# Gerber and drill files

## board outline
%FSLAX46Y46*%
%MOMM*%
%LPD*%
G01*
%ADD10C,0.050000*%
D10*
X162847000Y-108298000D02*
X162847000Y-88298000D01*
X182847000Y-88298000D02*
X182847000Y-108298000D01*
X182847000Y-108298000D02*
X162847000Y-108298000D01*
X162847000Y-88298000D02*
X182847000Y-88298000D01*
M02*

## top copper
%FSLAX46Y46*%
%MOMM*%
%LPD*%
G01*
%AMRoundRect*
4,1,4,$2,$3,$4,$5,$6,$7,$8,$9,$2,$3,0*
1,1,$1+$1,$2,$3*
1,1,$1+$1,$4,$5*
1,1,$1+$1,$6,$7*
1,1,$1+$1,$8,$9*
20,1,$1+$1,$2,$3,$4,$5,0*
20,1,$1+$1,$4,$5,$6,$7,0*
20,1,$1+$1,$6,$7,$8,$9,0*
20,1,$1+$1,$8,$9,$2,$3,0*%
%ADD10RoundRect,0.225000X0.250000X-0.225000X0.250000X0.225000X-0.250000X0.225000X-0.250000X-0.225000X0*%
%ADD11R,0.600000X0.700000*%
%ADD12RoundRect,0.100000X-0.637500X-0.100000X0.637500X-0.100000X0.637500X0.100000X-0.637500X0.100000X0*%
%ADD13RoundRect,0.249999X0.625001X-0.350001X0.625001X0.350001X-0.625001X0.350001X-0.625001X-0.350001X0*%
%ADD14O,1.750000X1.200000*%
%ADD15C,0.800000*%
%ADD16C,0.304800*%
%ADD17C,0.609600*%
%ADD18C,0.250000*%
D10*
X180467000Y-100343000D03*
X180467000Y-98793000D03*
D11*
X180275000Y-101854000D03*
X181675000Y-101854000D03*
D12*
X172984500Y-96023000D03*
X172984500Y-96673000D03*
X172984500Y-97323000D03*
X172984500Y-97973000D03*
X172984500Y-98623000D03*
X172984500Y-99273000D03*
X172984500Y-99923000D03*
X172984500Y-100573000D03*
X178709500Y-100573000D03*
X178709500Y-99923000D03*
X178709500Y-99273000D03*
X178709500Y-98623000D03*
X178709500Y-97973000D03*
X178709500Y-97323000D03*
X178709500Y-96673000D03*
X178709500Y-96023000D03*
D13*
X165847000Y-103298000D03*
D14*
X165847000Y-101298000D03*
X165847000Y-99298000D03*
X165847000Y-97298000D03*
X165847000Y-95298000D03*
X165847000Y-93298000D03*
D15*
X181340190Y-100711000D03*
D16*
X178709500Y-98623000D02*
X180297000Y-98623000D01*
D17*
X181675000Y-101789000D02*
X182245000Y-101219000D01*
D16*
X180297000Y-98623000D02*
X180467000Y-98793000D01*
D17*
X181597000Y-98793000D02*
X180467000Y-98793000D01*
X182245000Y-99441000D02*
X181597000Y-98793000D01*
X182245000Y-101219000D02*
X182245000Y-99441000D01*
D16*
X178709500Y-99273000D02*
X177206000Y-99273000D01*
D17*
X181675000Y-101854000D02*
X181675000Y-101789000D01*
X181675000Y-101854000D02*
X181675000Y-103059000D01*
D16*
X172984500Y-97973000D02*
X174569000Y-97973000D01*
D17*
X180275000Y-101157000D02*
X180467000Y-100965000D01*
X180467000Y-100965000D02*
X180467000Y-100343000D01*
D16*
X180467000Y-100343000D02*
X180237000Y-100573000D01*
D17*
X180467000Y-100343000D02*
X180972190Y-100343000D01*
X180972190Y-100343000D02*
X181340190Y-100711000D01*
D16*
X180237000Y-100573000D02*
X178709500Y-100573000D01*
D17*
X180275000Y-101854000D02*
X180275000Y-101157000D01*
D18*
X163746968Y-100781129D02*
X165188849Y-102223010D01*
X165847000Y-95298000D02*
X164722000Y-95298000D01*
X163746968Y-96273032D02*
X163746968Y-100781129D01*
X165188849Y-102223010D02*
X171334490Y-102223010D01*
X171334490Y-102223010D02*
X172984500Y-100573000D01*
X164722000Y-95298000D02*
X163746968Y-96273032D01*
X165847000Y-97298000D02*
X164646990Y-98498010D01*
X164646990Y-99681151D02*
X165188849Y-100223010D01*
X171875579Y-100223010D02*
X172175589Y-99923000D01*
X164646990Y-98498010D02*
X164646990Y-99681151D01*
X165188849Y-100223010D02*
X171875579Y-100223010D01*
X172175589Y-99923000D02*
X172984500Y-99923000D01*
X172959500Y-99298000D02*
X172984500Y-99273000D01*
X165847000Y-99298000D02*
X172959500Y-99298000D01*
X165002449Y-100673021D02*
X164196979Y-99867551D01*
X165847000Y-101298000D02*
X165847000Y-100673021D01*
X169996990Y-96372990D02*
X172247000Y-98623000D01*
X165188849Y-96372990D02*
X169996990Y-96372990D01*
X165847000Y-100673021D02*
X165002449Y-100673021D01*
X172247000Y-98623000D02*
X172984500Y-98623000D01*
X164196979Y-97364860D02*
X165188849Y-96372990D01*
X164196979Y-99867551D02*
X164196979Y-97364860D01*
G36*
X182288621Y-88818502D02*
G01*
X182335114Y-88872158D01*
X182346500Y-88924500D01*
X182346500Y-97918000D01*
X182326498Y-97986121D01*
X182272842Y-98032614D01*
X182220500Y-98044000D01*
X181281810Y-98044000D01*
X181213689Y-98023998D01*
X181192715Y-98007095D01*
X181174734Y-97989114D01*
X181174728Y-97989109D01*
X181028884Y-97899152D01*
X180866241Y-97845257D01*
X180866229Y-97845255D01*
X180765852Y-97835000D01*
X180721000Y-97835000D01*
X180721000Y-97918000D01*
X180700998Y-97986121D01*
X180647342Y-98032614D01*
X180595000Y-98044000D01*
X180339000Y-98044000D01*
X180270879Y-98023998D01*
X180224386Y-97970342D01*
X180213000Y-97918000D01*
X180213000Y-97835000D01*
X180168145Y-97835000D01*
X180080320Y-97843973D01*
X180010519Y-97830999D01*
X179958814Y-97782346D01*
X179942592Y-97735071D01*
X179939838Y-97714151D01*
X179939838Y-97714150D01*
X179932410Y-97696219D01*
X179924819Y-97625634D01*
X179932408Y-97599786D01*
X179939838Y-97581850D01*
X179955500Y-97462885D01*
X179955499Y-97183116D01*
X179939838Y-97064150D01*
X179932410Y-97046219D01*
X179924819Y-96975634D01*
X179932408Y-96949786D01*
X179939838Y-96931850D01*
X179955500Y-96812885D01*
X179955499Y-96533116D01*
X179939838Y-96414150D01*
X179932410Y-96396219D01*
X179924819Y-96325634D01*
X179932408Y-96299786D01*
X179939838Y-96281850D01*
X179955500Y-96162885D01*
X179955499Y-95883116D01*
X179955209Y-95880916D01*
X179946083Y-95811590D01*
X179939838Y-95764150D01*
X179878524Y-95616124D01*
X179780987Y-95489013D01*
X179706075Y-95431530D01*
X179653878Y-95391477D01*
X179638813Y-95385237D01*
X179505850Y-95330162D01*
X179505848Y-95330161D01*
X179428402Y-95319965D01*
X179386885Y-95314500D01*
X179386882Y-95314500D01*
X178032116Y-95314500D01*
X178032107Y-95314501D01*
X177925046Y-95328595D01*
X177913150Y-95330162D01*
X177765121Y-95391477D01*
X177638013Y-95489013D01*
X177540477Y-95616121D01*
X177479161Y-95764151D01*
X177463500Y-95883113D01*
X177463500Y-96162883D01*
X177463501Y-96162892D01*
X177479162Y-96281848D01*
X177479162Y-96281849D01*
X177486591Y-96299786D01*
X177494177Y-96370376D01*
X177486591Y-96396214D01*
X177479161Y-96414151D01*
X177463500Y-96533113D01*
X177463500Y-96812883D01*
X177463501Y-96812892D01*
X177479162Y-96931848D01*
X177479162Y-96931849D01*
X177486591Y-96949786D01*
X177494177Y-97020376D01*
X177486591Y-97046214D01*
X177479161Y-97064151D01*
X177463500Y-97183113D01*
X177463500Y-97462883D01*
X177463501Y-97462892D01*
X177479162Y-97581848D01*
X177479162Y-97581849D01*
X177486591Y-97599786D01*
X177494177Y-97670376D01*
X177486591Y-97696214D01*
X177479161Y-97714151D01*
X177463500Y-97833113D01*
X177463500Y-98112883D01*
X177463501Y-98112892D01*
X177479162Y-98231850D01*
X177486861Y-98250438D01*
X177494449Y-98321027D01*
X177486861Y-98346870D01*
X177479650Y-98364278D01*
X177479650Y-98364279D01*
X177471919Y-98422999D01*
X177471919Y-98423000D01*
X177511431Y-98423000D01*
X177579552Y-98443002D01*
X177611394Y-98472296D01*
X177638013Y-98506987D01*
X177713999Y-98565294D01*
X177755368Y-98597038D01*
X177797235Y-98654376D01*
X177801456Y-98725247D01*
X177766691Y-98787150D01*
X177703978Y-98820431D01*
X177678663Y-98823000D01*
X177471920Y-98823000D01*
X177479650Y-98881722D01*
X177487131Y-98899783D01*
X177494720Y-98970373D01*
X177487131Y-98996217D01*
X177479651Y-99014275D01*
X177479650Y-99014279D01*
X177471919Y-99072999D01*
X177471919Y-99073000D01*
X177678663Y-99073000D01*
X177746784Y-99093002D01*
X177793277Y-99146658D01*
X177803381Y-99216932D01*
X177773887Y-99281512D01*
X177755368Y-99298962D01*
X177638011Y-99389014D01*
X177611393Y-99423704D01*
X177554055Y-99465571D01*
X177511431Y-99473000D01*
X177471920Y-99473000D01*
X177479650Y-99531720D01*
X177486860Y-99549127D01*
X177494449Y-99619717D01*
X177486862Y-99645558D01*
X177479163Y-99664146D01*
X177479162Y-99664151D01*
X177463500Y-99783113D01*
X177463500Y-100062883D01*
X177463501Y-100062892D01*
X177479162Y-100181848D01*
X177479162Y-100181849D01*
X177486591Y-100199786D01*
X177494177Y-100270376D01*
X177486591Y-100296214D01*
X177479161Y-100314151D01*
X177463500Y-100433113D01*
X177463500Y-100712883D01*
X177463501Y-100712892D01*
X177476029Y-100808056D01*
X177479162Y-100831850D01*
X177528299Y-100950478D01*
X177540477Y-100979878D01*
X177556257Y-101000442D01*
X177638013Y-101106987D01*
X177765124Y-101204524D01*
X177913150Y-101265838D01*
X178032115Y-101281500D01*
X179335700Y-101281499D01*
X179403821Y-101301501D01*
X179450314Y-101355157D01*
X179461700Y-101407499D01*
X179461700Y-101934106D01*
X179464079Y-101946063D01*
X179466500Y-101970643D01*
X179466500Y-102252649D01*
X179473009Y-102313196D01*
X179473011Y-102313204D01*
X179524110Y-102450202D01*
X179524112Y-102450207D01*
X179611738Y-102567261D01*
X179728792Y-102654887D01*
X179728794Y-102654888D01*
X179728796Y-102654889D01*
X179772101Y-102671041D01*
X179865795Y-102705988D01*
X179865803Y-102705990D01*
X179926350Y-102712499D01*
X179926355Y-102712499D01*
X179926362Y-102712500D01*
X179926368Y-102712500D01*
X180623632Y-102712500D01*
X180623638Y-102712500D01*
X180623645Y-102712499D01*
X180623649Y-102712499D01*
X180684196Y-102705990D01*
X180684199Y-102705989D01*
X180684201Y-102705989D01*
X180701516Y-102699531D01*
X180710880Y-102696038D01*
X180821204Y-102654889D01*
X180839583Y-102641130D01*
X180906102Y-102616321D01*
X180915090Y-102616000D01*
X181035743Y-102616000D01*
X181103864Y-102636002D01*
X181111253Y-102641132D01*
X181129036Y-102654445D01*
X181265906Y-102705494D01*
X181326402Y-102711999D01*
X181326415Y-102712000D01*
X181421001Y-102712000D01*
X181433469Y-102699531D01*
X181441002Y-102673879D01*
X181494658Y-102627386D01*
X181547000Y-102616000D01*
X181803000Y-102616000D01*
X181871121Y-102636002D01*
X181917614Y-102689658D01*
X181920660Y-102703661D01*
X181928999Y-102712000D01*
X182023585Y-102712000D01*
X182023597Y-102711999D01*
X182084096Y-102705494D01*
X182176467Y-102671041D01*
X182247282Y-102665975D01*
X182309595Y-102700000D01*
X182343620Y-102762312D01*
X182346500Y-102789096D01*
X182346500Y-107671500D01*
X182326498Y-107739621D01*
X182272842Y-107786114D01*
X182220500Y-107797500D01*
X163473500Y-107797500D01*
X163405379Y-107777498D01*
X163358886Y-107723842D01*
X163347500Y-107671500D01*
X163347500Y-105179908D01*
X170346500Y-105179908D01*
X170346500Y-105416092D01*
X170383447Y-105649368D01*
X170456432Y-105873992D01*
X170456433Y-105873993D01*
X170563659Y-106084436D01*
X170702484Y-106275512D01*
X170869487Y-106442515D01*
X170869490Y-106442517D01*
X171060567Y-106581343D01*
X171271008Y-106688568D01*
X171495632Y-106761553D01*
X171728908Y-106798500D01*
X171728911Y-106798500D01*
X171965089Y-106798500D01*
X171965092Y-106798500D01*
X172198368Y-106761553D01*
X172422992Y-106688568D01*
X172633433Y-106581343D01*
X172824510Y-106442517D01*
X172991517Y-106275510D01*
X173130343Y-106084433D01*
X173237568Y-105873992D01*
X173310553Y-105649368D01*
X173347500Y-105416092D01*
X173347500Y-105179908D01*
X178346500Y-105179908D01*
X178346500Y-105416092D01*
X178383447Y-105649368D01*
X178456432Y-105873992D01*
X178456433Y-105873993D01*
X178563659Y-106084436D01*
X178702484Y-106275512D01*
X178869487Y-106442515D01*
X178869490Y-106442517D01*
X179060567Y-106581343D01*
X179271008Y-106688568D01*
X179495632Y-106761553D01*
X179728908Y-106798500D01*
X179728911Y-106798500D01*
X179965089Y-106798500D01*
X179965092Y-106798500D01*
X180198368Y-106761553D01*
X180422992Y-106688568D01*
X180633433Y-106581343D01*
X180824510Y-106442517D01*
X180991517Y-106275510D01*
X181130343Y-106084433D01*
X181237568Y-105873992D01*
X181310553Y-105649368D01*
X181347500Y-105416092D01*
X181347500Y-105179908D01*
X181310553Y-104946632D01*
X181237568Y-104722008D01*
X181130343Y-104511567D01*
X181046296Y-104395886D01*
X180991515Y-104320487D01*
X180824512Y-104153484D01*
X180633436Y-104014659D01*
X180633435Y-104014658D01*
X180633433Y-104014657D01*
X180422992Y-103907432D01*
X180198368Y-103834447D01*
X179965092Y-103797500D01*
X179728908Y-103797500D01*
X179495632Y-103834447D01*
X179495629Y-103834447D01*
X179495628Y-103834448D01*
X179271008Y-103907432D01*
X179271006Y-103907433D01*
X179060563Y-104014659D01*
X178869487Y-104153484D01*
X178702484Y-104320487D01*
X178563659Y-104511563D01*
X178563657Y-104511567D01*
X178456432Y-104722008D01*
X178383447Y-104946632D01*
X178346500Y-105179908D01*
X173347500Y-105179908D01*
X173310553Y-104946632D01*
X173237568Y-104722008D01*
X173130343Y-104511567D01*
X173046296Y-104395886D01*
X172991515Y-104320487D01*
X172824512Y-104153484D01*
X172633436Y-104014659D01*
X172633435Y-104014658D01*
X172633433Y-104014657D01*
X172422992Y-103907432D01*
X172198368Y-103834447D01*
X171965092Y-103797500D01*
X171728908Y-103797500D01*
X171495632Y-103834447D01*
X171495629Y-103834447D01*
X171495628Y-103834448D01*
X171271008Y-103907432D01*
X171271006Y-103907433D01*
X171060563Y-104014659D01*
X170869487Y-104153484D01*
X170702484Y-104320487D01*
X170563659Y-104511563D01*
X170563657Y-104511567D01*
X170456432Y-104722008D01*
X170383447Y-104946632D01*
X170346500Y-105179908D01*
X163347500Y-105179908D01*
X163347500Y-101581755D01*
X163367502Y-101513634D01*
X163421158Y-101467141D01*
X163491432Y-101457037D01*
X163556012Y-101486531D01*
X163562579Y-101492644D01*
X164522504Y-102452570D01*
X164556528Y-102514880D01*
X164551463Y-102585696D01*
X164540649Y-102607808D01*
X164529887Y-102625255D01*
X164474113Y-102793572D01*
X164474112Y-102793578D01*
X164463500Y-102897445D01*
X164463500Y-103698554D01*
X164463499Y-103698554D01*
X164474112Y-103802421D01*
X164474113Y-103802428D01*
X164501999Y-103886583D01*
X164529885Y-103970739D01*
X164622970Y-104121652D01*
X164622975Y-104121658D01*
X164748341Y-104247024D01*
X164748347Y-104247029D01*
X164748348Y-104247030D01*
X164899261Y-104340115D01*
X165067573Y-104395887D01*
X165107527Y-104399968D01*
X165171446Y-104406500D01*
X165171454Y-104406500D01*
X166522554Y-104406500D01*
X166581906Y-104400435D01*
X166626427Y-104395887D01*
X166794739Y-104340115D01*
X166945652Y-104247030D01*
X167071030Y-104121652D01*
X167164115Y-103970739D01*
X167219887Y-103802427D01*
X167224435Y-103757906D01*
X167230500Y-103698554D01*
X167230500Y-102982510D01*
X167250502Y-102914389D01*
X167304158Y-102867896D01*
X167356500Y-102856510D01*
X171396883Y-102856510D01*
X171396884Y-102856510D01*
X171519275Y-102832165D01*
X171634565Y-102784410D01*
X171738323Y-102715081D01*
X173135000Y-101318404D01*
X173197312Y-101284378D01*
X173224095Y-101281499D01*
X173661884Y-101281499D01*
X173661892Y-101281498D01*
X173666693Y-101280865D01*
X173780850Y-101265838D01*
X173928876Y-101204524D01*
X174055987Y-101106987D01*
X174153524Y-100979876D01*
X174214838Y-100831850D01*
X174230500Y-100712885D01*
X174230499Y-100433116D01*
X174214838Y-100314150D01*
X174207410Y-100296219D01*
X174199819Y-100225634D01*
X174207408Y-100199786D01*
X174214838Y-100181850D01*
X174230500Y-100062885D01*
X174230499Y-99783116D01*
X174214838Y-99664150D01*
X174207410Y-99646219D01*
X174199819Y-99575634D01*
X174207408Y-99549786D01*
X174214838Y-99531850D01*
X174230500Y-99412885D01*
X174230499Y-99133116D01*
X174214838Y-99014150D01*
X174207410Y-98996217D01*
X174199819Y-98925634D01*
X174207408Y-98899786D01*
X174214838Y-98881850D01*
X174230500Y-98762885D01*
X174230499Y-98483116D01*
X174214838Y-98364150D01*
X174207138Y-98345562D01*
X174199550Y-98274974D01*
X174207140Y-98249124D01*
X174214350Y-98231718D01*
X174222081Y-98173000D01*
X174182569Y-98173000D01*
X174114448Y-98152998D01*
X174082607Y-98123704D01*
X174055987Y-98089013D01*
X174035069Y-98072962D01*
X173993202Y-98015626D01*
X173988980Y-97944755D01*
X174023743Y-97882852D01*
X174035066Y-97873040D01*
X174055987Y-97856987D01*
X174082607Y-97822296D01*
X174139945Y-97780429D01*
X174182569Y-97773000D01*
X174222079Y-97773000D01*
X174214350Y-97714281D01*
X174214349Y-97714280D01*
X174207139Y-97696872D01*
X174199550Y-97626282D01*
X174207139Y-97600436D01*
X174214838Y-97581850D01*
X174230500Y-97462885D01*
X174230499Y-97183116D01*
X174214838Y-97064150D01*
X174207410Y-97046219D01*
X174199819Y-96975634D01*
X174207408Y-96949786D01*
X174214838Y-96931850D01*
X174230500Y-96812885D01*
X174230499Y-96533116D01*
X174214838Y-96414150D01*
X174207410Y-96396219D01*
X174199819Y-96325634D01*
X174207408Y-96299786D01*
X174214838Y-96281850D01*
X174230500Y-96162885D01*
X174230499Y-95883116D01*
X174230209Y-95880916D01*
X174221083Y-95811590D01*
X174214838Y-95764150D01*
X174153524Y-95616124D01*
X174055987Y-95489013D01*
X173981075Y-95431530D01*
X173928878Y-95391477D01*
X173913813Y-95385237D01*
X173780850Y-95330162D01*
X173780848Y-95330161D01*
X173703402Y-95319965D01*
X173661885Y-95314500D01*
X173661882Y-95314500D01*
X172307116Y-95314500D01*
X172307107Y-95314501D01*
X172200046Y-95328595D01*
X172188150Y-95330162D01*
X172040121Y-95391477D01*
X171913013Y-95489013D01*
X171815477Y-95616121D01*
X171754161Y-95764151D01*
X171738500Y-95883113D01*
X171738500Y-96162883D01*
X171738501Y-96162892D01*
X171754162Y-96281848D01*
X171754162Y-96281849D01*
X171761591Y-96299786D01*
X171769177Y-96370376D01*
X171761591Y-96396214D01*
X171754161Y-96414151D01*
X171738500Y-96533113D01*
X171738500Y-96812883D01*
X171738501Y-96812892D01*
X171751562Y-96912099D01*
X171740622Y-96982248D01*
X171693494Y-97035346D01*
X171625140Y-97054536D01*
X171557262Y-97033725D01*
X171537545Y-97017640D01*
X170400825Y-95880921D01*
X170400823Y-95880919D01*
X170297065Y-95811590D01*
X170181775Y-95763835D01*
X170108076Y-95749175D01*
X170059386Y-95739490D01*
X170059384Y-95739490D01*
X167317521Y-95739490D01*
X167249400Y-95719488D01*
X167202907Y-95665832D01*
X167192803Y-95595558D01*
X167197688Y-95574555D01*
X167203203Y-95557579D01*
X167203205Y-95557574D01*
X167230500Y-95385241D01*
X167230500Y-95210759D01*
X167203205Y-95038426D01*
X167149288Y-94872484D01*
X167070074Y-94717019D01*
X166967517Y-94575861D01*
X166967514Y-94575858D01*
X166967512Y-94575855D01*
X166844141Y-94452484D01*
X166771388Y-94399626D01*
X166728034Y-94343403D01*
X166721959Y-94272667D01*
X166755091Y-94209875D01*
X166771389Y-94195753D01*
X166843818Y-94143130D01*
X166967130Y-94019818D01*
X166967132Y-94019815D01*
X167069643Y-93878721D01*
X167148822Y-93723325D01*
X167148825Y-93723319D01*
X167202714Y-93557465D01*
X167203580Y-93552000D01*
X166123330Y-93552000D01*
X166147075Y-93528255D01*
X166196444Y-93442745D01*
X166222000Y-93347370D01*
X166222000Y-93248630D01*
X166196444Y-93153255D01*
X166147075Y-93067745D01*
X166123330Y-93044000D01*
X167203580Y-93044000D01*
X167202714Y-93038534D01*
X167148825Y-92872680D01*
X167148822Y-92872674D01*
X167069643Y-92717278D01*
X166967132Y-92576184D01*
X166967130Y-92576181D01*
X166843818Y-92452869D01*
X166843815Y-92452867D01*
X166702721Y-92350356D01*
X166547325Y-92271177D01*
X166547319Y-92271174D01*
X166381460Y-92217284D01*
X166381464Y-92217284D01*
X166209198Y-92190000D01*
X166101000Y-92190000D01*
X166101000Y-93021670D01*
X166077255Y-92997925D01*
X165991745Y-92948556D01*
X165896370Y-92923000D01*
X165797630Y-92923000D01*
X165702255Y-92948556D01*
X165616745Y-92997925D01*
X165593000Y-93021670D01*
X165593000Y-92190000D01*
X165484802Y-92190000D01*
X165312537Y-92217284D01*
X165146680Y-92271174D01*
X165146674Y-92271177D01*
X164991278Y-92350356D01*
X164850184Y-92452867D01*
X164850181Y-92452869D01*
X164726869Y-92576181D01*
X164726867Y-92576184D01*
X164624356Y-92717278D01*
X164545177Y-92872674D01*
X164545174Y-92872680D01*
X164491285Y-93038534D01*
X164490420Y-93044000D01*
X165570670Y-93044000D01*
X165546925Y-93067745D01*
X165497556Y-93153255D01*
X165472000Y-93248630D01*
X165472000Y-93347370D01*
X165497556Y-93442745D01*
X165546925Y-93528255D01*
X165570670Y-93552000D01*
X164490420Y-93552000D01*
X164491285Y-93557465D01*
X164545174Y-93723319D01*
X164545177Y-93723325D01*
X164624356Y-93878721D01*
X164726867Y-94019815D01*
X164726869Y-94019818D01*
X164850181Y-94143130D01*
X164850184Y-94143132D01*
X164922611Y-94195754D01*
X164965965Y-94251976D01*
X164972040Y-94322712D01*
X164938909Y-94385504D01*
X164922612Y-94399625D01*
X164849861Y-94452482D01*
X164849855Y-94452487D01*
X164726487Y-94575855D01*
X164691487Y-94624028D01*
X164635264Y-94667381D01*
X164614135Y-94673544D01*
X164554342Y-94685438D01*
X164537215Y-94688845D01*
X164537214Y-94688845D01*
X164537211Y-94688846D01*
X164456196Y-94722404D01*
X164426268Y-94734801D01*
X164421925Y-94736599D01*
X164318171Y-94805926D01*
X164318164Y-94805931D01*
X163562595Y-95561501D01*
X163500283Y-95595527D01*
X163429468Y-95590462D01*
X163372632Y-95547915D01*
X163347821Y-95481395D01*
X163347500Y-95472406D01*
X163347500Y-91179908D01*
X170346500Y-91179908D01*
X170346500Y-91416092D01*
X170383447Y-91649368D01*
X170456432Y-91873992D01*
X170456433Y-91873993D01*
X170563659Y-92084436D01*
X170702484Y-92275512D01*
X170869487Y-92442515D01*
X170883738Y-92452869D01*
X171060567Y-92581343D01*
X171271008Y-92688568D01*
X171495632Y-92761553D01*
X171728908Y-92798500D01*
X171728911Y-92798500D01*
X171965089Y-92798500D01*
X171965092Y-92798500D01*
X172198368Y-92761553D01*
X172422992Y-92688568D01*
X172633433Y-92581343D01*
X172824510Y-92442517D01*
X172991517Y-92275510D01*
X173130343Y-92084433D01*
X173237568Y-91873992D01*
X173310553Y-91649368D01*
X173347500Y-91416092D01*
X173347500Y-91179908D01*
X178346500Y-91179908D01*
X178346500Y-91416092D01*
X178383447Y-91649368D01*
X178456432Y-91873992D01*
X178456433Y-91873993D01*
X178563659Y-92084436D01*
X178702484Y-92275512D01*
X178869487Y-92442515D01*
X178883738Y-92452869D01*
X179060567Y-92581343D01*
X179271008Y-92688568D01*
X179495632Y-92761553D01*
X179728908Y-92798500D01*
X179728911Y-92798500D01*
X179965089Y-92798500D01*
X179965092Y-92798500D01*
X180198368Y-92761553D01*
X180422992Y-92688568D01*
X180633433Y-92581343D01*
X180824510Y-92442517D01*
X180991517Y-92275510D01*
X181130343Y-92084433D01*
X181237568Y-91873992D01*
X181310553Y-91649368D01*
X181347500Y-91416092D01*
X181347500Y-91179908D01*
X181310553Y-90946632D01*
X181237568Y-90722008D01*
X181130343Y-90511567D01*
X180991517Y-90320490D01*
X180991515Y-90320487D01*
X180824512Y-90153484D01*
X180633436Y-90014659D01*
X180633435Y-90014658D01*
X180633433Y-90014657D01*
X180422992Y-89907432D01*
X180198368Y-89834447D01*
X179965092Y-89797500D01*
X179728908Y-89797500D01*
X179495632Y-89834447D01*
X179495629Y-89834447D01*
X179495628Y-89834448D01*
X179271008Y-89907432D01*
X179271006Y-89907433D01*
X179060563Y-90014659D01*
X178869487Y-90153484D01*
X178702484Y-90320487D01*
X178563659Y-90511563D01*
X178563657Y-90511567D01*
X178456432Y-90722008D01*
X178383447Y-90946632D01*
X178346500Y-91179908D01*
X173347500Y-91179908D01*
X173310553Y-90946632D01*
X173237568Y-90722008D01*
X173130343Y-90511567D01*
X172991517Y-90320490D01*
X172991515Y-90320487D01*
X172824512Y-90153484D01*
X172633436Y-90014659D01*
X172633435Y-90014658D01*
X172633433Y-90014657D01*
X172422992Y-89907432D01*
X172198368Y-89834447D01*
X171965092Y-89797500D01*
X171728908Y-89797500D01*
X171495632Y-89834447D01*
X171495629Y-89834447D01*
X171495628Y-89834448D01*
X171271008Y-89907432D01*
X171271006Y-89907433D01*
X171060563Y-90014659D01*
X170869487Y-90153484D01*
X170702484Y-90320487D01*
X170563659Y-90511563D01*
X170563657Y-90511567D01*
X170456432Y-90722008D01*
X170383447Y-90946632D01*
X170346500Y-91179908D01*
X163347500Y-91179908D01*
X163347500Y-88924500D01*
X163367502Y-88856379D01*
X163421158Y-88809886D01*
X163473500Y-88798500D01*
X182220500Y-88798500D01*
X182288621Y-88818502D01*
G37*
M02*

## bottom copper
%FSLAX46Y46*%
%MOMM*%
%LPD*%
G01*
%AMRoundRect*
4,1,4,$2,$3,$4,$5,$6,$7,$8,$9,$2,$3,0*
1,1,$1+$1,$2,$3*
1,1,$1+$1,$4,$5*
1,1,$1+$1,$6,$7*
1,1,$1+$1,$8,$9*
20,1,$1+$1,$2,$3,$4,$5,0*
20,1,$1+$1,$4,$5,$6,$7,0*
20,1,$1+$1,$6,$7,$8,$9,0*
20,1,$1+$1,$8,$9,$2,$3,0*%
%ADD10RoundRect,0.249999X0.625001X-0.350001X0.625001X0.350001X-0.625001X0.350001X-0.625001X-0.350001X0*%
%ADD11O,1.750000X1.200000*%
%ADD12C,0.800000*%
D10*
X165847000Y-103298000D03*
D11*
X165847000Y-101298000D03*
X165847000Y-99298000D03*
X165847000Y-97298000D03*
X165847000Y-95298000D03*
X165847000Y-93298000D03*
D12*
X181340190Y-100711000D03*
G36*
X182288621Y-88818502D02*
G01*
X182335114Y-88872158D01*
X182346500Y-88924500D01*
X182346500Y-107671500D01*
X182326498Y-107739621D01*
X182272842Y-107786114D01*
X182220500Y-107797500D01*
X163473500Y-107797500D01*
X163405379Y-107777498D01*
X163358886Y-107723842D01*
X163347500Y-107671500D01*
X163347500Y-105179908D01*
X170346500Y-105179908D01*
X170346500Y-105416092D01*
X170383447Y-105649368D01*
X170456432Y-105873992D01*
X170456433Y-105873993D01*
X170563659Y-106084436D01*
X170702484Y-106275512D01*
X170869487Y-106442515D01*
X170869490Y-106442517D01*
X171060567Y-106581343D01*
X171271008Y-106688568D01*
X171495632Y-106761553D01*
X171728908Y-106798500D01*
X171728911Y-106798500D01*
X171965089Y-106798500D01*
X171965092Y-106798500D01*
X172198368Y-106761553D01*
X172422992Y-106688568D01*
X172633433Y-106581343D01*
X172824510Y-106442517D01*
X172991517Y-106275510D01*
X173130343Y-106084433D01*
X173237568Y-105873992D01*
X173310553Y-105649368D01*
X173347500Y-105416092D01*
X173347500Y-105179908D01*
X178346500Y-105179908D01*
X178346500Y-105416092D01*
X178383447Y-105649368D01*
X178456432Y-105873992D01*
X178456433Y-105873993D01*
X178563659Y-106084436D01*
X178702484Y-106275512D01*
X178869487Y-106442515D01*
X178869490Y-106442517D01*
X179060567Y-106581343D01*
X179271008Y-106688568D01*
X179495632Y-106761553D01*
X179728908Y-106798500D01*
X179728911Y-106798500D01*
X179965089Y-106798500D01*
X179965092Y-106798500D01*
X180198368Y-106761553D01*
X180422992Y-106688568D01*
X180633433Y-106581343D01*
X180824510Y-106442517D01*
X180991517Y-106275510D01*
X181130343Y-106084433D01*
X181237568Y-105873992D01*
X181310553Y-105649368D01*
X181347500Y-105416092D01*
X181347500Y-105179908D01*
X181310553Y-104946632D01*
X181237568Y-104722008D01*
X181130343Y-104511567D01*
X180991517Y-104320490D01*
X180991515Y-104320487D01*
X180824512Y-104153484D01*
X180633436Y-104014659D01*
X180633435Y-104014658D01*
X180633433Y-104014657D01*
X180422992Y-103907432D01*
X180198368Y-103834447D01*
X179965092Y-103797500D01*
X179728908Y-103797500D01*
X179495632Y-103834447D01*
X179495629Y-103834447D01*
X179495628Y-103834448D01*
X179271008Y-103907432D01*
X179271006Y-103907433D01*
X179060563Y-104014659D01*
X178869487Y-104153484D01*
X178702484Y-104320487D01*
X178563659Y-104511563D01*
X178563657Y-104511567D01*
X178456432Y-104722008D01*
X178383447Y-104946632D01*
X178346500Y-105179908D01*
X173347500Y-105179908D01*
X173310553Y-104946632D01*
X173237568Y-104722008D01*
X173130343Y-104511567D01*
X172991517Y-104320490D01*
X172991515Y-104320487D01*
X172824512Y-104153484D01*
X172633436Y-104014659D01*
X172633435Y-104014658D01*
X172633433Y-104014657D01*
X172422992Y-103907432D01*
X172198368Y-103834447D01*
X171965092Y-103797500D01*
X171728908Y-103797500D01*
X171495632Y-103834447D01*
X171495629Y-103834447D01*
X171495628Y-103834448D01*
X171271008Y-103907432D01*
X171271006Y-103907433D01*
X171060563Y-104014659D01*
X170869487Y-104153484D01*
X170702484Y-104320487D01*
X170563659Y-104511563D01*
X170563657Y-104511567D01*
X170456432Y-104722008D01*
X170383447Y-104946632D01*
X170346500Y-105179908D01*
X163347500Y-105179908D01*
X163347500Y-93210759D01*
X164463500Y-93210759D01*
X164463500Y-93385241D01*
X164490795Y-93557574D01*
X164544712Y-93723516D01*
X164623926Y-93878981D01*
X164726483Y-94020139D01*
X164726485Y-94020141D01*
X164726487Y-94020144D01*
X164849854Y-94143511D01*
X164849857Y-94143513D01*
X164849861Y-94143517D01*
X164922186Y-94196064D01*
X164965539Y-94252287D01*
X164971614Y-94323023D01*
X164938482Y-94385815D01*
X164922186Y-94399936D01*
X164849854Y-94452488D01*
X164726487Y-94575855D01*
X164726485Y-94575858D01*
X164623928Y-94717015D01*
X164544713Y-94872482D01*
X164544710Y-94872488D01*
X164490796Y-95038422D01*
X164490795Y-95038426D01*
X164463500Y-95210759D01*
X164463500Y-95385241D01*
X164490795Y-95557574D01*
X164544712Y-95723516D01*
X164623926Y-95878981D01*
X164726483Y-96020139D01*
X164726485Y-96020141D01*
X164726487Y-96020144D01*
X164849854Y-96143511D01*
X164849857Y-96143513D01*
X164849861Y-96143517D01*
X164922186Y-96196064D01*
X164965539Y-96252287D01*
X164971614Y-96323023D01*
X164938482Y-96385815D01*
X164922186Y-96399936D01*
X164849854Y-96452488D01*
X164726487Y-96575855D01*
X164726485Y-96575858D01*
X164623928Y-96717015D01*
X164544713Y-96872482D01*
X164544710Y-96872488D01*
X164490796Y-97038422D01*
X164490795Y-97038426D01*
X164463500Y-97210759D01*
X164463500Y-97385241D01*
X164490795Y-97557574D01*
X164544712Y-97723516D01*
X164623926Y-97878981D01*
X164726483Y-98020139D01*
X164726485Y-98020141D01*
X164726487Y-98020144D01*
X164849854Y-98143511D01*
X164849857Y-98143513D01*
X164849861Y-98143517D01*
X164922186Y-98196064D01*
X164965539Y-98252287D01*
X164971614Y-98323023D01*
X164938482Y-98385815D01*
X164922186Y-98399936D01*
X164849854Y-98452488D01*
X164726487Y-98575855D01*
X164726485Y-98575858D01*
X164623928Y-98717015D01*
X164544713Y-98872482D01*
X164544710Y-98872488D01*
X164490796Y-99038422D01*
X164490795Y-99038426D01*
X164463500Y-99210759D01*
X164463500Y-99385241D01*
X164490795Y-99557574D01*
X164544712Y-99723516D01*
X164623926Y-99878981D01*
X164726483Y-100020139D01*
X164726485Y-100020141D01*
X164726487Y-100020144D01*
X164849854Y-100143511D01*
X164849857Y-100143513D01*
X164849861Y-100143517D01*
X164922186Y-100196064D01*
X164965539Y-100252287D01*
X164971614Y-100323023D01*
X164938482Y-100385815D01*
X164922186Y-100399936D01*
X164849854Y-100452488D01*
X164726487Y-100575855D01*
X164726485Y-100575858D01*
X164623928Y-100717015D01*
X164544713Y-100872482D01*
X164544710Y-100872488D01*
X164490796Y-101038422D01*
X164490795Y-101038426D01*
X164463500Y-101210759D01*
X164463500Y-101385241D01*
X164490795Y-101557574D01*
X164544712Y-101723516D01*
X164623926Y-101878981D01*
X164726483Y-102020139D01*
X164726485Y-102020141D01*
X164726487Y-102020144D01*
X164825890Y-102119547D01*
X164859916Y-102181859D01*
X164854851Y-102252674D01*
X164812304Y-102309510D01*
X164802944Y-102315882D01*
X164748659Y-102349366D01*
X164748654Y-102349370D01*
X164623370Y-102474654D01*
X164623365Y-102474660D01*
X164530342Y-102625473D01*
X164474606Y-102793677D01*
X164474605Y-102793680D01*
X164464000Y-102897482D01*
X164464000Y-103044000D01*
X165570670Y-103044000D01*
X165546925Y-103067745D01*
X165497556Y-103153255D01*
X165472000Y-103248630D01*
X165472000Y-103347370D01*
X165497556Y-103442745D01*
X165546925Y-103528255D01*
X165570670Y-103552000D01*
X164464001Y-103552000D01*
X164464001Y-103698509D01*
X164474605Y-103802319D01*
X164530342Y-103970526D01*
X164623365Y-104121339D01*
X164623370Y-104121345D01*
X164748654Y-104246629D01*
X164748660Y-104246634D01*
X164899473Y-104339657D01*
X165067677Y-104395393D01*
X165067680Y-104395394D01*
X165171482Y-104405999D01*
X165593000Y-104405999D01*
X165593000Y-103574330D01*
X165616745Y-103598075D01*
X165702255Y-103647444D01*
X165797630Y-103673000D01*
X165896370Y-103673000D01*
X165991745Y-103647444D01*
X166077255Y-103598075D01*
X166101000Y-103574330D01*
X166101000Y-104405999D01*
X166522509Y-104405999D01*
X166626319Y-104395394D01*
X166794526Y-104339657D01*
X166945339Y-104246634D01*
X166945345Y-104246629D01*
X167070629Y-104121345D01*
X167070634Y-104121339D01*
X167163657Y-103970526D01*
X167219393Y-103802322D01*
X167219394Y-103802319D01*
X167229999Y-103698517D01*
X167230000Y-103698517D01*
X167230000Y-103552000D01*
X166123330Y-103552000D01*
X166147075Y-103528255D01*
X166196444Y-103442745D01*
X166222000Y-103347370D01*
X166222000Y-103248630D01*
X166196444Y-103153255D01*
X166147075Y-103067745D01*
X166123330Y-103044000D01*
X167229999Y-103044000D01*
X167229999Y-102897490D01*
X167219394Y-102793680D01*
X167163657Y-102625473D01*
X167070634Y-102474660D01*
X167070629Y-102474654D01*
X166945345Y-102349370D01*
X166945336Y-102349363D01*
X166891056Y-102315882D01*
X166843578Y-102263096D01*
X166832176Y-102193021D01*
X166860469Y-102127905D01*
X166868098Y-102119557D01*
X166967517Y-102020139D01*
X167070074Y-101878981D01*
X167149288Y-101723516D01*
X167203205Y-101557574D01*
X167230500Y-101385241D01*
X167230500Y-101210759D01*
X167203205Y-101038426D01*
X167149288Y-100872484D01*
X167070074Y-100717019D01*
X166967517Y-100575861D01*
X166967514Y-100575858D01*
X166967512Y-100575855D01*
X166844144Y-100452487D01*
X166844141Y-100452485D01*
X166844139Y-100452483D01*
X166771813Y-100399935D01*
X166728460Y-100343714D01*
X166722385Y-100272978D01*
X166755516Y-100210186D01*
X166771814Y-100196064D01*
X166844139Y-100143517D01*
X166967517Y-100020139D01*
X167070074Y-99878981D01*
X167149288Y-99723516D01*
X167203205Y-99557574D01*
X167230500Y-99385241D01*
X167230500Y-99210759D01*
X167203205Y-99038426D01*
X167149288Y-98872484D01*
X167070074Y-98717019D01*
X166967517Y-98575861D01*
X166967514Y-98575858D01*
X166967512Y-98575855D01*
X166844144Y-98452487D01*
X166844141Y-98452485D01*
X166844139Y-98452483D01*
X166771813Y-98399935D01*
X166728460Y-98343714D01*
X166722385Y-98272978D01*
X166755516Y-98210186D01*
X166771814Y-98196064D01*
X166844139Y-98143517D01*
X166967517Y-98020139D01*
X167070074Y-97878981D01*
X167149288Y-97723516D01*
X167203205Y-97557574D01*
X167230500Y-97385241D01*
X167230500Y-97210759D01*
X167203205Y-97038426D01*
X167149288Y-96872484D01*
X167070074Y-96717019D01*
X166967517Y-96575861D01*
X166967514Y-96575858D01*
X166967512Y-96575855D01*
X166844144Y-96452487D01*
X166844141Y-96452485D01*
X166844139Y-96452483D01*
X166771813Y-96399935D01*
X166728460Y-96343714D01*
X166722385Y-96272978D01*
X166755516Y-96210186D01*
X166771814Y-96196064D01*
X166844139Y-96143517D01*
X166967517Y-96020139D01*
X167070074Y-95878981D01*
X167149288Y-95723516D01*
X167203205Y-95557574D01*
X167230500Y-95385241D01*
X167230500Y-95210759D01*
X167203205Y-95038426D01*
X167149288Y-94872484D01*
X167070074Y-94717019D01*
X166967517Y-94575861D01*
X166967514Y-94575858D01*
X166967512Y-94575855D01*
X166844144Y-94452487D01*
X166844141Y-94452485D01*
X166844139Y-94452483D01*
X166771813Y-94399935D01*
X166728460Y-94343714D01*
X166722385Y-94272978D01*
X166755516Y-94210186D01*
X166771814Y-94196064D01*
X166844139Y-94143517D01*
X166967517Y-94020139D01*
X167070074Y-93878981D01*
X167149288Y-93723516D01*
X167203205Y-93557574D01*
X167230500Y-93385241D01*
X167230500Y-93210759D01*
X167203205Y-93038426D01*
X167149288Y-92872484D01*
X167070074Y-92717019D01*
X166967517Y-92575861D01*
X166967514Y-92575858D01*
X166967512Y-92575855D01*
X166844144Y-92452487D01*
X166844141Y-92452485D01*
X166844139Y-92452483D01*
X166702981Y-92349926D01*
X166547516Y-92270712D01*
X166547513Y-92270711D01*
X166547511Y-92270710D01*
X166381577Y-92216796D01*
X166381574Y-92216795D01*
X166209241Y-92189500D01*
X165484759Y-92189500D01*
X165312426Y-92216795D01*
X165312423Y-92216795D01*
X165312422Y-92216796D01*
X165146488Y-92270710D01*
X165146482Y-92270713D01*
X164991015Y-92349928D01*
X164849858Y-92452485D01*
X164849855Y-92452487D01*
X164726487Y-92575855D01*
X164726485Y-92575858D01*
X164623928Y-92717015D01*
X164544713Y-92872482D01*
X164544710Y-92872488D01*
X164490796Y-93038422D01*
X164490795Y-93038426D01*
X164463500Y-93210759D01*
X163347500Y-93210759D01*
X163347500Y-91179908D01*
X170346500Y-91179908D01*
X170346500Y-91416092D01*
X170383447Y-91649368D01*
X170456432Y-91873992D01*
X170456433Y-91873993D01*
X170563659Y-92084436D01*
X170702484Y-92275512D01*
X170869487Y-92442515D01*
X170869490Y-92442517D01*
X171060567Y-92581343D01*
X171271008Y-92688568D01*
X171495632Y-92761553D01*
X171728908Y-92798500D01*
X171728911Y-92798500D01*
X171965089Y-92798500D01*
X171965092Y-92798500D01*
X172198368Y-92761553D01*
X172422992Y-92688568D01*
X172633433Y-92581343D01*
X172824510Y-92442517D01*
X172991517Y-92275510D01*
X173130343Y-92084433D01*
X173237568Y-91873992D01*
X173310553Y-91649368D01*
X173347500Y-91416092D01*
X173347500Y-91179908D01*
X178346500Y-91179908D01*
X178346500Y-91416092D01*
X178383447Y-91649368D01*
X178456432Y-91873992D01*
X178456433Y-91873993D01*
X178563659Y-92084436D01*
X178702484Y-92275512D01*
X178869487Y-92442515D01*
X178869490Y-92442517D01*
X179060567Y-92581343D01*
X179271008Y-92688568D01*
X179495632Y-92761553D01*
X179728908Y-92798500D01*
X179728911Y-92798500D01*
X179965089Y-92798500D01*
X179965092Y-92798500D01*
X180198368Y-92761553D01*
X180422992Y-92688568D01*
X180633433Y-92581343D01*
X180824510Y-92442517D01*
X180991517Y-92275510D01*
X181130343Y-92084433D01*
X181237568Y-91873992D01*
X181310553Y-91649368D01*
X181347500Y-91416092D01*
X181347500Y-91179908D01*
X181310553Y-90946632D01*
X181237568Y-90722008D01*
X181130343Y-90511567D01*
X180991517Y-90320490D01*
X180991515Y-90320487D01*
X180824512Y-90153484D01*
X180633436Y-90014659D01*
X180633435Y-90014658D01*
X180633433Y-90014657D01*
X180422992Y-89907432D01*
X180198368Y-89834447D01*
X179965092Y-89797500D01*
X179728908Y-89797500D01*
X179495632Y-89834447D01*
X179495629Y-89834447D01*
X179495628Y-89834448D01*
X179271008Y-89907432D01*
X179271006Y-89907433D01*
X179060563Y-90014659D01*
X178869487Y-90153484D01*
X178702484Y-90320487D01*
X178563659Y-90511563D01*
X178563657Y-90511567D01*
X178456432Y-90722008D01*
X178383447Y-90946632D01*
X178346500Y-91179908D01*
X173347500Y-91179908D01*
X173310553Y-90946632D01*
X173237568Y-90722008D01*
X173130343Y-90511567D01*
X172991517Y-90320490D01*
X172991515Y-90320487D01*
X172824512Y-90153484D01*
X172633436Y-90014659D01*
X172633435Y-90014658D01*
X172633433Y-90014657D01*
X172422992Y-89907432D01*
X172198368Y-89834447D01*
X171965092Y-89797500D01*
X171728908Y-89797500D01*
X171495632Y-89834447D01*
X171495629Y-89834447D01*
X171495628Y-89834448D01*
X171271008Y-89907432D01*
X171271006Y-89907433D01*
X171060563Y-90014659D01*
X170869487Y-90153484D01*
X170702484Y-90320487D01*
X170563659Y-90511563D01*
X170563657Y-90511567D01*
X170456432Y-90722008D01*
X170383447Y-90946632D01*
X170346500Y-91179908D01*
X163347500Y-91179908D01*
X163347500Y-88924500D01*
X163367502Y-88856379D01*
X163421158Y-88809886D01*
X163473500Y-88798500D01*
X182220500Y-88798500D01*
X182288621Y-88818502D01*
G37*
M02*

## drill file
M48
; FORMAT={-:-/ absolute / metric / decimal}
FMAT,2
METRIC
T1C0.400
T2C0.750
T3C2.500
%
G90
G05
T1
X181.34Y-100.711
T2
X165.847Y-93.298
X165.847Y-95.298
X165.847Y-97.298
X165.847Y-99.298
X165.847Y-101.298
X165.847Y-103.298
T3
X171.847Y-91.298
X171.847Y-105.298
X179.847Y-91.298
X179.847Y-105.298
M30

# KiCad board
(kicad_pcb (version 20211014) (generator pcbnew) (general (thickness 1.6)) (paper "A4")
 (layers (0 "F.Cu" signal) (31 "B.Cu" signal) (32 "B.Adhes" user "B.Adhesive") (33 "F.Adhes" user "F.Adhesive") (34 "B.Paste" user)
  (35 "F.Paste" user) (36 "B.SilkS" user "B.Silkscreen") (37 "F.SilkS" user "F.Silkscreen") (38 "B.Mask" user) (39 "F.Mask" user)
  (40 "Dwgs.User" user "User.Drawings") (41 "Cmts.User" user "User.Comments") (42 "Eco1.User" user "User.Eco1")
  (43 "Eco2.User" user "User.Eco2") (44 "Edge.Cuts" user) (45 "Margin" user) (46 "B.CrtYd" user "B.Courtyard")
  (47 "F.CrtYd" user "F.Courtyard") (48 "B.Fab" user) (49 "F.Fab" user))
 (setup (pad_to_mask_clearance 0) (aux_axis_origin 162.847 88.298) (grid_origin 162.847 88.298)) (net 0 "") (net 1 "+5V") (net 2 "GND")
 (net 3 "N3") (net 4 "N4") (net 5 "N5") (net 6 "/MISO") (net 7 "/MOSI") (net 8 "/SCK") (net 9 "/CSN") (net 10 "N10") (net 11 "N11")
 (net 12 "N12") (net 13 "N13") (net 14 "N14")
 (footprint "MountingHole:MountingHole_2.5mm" (layer "F.Cu") (at 179.847 91.298)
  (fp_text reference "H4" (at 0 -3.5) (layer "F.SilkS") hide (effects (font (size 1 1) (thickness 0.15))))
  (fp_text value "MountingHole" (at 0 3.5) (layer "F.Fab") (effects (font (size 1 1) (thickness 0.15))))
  (pad "" np_thru_hole circle locked (at 0 0) (size 2.5 2.5) (drill 2.5) (layers *.Cu *.Mask)))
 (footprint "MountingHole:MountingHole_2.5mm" (layer "F.Cu") (at 179.847 105.298)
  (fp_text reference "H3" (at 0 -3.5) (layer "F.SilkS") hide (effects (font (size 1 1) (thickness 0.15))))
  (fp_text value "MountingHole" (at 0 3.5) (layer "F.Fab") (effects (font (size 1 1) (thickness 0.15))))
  (pad "" np_thru_hole circle locked (at 0 0) (size 2.5 2.5) (drill 2.5) (layers *.Cu *.Mask)))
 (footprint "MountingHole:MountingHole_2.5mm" (layer "F.Cu") (at 171.847 91.298)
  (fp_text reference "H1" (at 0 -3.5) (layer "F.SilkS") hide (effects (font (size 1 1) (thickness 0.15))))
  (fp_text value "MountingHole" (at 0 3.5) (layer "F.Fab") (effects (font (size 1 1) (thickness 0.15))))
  (pad "" np_thru_hole circle locked (at 0 0) (size 2.5 2.5) (drill 2.5) (layers *.Cu *.Mask)))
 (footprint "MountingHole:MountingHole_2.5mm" (layer "F.Cu") (at 171.847 105.298)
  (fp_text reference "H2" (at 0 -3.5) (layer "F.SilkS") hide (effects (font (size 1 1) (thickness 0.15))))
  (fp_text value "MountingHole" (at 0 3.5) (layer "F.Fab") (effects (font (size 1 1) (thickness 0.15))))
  (pad "" np_thru_hole circle locked (at 0 0) (size 2.5 2.5) (drill 2.5) (layers *.Cu *.Mask)))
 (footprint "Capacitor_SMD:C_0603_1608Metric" (layer "F.Cu") (at 180.467 99.568 90)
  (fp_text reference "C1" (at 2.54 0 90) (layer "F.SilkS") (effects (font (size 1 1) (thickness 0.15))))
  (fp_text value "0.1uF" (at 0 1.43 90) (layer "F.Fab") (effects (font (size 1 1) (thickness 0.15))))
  (pad "1" smd roundrect locked (at -0.775 0 90) (size 0.9 0.95) (layers "F.Cu" "F.Paste" "F.Mask") (roundrect_rratio 0.25) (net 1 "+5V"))
  (pad "2" smd roundrect locked (at 0.775 0 90) (size 0.9 0.95) (layers "F.Cu" "F.Paste" "F.Mask") (roundrect_rratio 0.25) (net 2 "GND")))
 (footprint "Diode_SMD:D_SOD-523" (layer "F.Cu") (at 180.975 101.854)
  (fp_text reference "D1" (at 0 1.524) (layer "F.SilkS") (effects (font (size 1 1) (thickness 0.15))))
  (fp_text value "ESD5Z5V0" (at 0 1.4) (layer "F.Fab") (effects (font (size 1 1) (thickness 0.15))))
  (pad "1" smd rect locked (at -0.7 0 180) (size 0.6 0.7) (layers "F.Cu" "F.Paste" "F.Mask") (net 1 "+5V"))
  (pad "2" smd rect locked (at 0.7 0 180) (size 0.6 0.7) (layers "F.Cu" "F.Paste" "F.Mask") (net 2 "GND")))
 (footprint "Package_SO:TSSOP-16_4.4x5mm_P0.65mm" (layer "F.Cu") (at 175.847 98.298)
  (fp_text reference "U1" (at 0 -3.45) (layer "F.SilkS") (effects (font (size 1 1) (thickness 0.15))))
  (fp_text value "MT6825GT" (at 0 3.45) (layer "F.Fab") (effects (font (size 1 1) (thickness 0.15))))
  (pad "1" smd roundrect locked (at -2.8625 -2.275) (size 1.475 0.4) (layers "F.Cu" "F.Paste" "F.Mask") (roundrect_rratio 0.25) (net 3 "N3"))
  (pad "2" smd roundrect locked (at -2.8625 -1.625) (size 1.475 0.4) (layers "F.Cu" "F.Paste" "F.Mask") (roundrect_rratio 0.25) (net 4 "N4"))
  (pad "3" smd roundrect locked (at -2.8625 -0.975) (size 1.475 0.4) (layers "F.Cu" "F.Paste" "F.Mask") (roundrect_rratio 0.25) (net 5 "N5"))
  (pad "4" smd roundrect locked (at -2.8625 -0.325) (size 1.475 0.4) (layers "F.Cu" "F.Paste" "F.Mask") (roundrect_rratio 0.25)
   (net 2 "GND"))
  (pad "5" smd roundrect locked (at -2.8625 0.325) (size 1.475 0.4) (layers "F.Cu" "F.Paste" "F.Mask") (roundrect_rratio 0.25)
   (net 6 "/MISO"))
  (pad "6" smd roundrect locked (at -2.8625 0.975) (size 1.475 0.4) (layers "F.Cu" "F.Paste" "F.Mask") (roundrect_rratio 0.25)
   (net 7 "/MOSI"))
  (pad "7" smd roundrect locked (at -2.8625 1.625) (size 1.475 0.4) (layers "F.Cu" "F.Paste" "F.Mask") (roundrect_rratio 0.25)
   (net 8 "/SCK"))
  (pad "8" smd roundrect locked (at -2.8625 2.275) (size 1.475 0.4) (layers "F.Cu" "F.Paste" "F.Mask") (roundrect_rratio 0.25)
   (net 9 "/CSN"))
  (pad "9" smd roundrect locked (at 2.8625 2.275) (size 1.475 0.4) (layers "F.Cu" "F.Paste" "F.Mask") (roundrect_rratio 0.25) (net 1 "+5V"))
  (pad "10" smd roundrect locked (at 2.8625 1.625) (size 1.475 0.4) (layers "F.Cu" "F.Paste" "F.Mask") (roundrect_rratio 0.25)
   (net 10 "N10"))
  (pad "11" smd roundrect locked (at 2.8625 0.975) (size 1.475 0.4) (layers "F.Cu" "F.Paste" "F.Mask") (roundrect_rratio 0.25) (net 2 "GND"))
  (pad "12" smd roundrect locked (at 2.8625 0.325) (size 1.475 0.4) (layers "F.Cu" "F.Paste" "F.Mask") (roundrect_rratio 0.25) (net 2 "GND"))
  (pad "13" smd roundrect locked (at 2.8625 -0.325) (size 1.475 0.4) (layers "F.Cu" "F.Paste" "F.Mask") (roundrect_rratio 0.25)
   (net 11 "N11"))
  (pad "14" smd roundrect locked (at 2.8625 -0.975) (size 1.475 0.4) (layers "F.Cu" "F.Paste" "F.Mask") (roundrect_rratio 0.25)
   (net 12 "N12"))
  (pad "15" smd roundrect locked (at 2.8625 -1.625) (size 1.475 0.4) (layers "F.Cu" "F.Paste" "F.Mask") (roundrect_rratio 0.25)
   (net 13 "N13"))
  (pad "16" smd roundrect locked (at 2.8625 -2.275) (size 1.475 0.4) (layers "F.Cu" "F.Paste" "F.Mask") (roundrect_rratio 0.25)
   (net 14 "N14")))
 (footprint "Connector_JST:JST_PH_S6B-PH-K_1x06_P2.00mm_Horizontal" (layer "B.Cu") (at 165.847 103.298 90)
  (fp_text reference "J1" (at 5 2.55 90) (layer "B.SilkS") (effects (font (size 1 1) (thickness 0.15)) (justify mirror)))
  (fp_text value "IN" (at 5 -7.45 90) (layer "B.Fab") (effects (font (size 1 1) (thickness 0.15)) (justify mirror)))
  (pad "1" thru_hole roundrect locked (at 0 0 90) (size 1.2 1.75) (drill 0.75) (layers *.Cu *.Mask) (roundrect_rratio 0.2083325)
   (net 1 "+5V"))
  (pad "2" thru_hole oval locked (at 2 0 90) (size 1.2 1.75) (drill 0.75) (layers *.Cu *.Mask) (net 6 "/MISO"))
  (pad "3" thru_hole oval locked (at 4 0 90) (size 1.2 1.75) (drill 0.75) (layers *.Cu *.Mask) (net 7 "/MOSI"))
  (pad "4" thru_hole oval locked (at 6 0 90) (size 1.2 1.75) (drill 0.75) (layers *.Cu *.Mask) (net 8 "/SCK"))
  (pad "5" thru_hole oval locked (at 8 0 90) (size 1.2 1.75) (drill 0.75) (layers *.Cu *.Mask) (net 9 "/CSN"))
  (pad "6" thru_hole oval locked (at 10 0 90) (size 1.2 1.75) (drill 0.75) (layers *.Cu *.Mask) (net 2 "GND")))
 (gr_line (start 162.847 108.298) (end 162.847 88.298) (layer "Edge.Cuts") (width 0.05))
 (gr_line (start 182.847 88.298) (end 182.847 108.298) (layer "Edge.Cuts") (width 0.05))
 (gr_line (start 182.847 108.298) (end 162.847 108.298) (layer "Edge.Cuts") (width 0.05))
 (gr_line (start 162.847 88.298) (end 182.847 88.298) (layer "Edge.Cuts") (width 0.05))
 (segment (start 178.7095 98.623) (end 180.297 98.623) (width 0.3048) (layer "F.Cu") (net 2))
 (segment (start 181.675 101.789) (end 182.245 101.219) (width 0.6096) (layer "F.Cu") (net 2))
 (segment (start 180.297 98.623) (end 180.467 98.793) (width 0.3048) (layer "F.Cu") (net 2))
 (segment (start 181.597 98.793) (end 180.467 98.793) (width 0.6096) (layer "F.Cu") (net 2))
 (segment (start 182.245 99.441) (end 181.597 98.793) (width 0.6096) (layer "F.Cu") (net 2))
 (segment (start 182.245 101.219) (end 182.245 99.441) (width 0.6096) (layer "F.Cu") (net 2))
 (segment (start 178.7095 99.273) (end 177.206 99.273) (width 0.3048) (layer "F.Cu") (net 2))
 (segment (start 181.675 101.854) (end 181.675 101.789) (width 0.6096) (layer "F.Cu") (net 2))
 (segment (start 181.675 101.854) (end 181.675 103.059) (width 0.6096) (layer "F.Cu") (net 2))
 (segment (start 172.9845 97.973) (end 174.569 97.973) (width 0.3048) (layer "F.Cu") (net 2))
 (segment (start 180.275 101.157) (end 180.467 100.965) (width 0.6096) (layer "F.Cu") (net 1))
 (segment (start 180.467 100.965) (end 180.467 100.343) (width 0.6096) (layer "F.Cu") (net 1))
 (segment (start 180.467 100.343) (end 180.237 100.573) (width 0.3048) (layer "F.Cu") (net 1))
 (segment (start 180.467 100.343) (end 180.97219 100.343) (width 0.6096) (layer "F.Cu") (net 1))
 (segment (start 180.97219 100.343) (end 181.34019 100.711) (width 0.6096) (layer "F.Cu") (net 1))
 (segment (start 180.237 100.573) (end 178.7095 100.573) (width 0.3048) (layer "F.Cu") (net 1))
 (segment (start 180.275 101.854) (end 180.275 101.157) (width 0.6096) (layer "F.Cu") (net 1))
 (via (at 181.34019 100.711) (size 0.8) (drill 0.4) (layers "F.Cu" "B.Cu") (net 1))
 (segment (start 163.746968 100.781129) (end 165.188849 102.22301) (width 0.25) (layer "F.Cu") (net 9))
 (segment (start 165.847 95.298) (end 164.722 95.298) (width 0.25) (layer "F.Cu") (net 9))
 (segment (start 163.746968 96.273032) (end 163.746968 100.781129) (width 0.25) (layer "F.Cu") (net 9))
 (segment (start 165.188849 102.22301) (end 171.33449 102.22301) (width 0.25) (layer "F.Cu") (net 9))
 (segment (start 171.33449 102.22301) (end 172.9845 100.573) (width 0.25) (layer "F.Cu") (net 9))
 (segment (start 164.722 95.298) (end 163.746968 96.273032) (width 0.25) (layer "F.Cu") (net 9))
 (segment (start 165.847 97.298) (end 164.64699 98.49801) (width 0.25) (layer "F.Cu") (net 8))
 (segment (start 164.64699 99.681151) (end 165.188849 100.22301) (width 0.25) (layer "F.Cu") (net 8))
 (segment (start 171.875579 100.22301) (end 172.175589 99.923) (width 0.25) (layer "F.Cu") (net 8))
 (segment (start 164.64699 98.49801) (end 164.64699 99.681151) (width 0.25) (layer "F.Cu") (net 8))
 (segment (start 165.188849 100.22301) (end 171.875579 100.22301) (width 0.25) (layer "F.Cu") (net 8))
 (segment (start 172.175589 99.923) (end 172.9845 99.923) (width 0.25) (layer "F.Cu") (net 8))
 (segment (start 172.9595 99.298) (end 172.9845 99.273) (width 0.25) (layer "F.Cu") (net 7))
 (segment (start 165.847 99.298) (end 172.9595 99.298) (width 0.25) (layer "F.Cu") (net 7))
 (segment (start 165.002449 100.673021) (end 164.196979 99.867551) (width 0.25) (layer "F.Cu") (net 6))
 (segment (start 165.847 101.298) (end 165.847 100.673021) (width 0.25) (layer "F.Cu") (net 6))
 (segment (start 169.99699 96.37299) (end 172.247 98.623) (width 0.25) (layer "F.Cu") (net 6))
 (segment (start 165.188849 96.37299) (end 169.99699 96.37299) (width 0.25) (layer "F.Cu") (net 6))
 (segment (start 165.847 100.673021) (end 165.002449 100.673021) (width 0.25) (layer "F.Cu") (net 6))
 (segment (start 172.247 98.623) (end 172.9845 98.623) (width 0.25) (layer "F.Cu") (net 6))
 (segment (start 164.196979 97.36486) (end 165.188849 96.37299) (width 0.25) (layer "F.Cu") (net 6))
 (segment (start 164.196979 99.867551) (end 164.196979 97.36486) (width 0.25) (layer "F.Cu") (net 6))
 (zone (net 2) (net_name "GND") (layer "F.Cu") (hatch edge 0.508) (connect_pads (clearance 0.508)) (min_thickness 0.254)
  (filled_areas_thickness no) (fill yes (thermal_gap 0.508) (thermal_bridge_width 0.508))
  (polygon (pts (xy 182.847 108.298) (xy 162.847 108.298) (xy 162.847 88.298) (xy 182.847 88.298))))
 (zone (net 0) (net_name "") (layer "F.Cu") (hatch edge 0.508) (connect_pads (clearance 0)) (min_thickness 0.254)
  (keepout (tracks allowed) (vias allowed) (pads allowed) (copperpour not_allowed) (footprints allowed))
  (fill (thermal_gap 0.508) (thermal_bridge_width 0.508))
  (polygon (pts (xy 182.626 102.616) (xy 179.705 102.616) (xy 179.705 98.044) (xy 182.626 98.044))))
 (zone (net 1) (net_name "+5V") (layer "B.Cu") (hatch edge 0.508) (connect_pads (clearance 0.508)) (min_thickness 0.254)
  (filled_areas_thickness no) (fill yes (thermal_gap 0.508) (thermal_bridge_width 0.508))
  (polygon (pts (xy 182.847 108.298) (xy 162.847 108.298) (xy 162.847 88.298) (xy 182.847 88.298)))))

